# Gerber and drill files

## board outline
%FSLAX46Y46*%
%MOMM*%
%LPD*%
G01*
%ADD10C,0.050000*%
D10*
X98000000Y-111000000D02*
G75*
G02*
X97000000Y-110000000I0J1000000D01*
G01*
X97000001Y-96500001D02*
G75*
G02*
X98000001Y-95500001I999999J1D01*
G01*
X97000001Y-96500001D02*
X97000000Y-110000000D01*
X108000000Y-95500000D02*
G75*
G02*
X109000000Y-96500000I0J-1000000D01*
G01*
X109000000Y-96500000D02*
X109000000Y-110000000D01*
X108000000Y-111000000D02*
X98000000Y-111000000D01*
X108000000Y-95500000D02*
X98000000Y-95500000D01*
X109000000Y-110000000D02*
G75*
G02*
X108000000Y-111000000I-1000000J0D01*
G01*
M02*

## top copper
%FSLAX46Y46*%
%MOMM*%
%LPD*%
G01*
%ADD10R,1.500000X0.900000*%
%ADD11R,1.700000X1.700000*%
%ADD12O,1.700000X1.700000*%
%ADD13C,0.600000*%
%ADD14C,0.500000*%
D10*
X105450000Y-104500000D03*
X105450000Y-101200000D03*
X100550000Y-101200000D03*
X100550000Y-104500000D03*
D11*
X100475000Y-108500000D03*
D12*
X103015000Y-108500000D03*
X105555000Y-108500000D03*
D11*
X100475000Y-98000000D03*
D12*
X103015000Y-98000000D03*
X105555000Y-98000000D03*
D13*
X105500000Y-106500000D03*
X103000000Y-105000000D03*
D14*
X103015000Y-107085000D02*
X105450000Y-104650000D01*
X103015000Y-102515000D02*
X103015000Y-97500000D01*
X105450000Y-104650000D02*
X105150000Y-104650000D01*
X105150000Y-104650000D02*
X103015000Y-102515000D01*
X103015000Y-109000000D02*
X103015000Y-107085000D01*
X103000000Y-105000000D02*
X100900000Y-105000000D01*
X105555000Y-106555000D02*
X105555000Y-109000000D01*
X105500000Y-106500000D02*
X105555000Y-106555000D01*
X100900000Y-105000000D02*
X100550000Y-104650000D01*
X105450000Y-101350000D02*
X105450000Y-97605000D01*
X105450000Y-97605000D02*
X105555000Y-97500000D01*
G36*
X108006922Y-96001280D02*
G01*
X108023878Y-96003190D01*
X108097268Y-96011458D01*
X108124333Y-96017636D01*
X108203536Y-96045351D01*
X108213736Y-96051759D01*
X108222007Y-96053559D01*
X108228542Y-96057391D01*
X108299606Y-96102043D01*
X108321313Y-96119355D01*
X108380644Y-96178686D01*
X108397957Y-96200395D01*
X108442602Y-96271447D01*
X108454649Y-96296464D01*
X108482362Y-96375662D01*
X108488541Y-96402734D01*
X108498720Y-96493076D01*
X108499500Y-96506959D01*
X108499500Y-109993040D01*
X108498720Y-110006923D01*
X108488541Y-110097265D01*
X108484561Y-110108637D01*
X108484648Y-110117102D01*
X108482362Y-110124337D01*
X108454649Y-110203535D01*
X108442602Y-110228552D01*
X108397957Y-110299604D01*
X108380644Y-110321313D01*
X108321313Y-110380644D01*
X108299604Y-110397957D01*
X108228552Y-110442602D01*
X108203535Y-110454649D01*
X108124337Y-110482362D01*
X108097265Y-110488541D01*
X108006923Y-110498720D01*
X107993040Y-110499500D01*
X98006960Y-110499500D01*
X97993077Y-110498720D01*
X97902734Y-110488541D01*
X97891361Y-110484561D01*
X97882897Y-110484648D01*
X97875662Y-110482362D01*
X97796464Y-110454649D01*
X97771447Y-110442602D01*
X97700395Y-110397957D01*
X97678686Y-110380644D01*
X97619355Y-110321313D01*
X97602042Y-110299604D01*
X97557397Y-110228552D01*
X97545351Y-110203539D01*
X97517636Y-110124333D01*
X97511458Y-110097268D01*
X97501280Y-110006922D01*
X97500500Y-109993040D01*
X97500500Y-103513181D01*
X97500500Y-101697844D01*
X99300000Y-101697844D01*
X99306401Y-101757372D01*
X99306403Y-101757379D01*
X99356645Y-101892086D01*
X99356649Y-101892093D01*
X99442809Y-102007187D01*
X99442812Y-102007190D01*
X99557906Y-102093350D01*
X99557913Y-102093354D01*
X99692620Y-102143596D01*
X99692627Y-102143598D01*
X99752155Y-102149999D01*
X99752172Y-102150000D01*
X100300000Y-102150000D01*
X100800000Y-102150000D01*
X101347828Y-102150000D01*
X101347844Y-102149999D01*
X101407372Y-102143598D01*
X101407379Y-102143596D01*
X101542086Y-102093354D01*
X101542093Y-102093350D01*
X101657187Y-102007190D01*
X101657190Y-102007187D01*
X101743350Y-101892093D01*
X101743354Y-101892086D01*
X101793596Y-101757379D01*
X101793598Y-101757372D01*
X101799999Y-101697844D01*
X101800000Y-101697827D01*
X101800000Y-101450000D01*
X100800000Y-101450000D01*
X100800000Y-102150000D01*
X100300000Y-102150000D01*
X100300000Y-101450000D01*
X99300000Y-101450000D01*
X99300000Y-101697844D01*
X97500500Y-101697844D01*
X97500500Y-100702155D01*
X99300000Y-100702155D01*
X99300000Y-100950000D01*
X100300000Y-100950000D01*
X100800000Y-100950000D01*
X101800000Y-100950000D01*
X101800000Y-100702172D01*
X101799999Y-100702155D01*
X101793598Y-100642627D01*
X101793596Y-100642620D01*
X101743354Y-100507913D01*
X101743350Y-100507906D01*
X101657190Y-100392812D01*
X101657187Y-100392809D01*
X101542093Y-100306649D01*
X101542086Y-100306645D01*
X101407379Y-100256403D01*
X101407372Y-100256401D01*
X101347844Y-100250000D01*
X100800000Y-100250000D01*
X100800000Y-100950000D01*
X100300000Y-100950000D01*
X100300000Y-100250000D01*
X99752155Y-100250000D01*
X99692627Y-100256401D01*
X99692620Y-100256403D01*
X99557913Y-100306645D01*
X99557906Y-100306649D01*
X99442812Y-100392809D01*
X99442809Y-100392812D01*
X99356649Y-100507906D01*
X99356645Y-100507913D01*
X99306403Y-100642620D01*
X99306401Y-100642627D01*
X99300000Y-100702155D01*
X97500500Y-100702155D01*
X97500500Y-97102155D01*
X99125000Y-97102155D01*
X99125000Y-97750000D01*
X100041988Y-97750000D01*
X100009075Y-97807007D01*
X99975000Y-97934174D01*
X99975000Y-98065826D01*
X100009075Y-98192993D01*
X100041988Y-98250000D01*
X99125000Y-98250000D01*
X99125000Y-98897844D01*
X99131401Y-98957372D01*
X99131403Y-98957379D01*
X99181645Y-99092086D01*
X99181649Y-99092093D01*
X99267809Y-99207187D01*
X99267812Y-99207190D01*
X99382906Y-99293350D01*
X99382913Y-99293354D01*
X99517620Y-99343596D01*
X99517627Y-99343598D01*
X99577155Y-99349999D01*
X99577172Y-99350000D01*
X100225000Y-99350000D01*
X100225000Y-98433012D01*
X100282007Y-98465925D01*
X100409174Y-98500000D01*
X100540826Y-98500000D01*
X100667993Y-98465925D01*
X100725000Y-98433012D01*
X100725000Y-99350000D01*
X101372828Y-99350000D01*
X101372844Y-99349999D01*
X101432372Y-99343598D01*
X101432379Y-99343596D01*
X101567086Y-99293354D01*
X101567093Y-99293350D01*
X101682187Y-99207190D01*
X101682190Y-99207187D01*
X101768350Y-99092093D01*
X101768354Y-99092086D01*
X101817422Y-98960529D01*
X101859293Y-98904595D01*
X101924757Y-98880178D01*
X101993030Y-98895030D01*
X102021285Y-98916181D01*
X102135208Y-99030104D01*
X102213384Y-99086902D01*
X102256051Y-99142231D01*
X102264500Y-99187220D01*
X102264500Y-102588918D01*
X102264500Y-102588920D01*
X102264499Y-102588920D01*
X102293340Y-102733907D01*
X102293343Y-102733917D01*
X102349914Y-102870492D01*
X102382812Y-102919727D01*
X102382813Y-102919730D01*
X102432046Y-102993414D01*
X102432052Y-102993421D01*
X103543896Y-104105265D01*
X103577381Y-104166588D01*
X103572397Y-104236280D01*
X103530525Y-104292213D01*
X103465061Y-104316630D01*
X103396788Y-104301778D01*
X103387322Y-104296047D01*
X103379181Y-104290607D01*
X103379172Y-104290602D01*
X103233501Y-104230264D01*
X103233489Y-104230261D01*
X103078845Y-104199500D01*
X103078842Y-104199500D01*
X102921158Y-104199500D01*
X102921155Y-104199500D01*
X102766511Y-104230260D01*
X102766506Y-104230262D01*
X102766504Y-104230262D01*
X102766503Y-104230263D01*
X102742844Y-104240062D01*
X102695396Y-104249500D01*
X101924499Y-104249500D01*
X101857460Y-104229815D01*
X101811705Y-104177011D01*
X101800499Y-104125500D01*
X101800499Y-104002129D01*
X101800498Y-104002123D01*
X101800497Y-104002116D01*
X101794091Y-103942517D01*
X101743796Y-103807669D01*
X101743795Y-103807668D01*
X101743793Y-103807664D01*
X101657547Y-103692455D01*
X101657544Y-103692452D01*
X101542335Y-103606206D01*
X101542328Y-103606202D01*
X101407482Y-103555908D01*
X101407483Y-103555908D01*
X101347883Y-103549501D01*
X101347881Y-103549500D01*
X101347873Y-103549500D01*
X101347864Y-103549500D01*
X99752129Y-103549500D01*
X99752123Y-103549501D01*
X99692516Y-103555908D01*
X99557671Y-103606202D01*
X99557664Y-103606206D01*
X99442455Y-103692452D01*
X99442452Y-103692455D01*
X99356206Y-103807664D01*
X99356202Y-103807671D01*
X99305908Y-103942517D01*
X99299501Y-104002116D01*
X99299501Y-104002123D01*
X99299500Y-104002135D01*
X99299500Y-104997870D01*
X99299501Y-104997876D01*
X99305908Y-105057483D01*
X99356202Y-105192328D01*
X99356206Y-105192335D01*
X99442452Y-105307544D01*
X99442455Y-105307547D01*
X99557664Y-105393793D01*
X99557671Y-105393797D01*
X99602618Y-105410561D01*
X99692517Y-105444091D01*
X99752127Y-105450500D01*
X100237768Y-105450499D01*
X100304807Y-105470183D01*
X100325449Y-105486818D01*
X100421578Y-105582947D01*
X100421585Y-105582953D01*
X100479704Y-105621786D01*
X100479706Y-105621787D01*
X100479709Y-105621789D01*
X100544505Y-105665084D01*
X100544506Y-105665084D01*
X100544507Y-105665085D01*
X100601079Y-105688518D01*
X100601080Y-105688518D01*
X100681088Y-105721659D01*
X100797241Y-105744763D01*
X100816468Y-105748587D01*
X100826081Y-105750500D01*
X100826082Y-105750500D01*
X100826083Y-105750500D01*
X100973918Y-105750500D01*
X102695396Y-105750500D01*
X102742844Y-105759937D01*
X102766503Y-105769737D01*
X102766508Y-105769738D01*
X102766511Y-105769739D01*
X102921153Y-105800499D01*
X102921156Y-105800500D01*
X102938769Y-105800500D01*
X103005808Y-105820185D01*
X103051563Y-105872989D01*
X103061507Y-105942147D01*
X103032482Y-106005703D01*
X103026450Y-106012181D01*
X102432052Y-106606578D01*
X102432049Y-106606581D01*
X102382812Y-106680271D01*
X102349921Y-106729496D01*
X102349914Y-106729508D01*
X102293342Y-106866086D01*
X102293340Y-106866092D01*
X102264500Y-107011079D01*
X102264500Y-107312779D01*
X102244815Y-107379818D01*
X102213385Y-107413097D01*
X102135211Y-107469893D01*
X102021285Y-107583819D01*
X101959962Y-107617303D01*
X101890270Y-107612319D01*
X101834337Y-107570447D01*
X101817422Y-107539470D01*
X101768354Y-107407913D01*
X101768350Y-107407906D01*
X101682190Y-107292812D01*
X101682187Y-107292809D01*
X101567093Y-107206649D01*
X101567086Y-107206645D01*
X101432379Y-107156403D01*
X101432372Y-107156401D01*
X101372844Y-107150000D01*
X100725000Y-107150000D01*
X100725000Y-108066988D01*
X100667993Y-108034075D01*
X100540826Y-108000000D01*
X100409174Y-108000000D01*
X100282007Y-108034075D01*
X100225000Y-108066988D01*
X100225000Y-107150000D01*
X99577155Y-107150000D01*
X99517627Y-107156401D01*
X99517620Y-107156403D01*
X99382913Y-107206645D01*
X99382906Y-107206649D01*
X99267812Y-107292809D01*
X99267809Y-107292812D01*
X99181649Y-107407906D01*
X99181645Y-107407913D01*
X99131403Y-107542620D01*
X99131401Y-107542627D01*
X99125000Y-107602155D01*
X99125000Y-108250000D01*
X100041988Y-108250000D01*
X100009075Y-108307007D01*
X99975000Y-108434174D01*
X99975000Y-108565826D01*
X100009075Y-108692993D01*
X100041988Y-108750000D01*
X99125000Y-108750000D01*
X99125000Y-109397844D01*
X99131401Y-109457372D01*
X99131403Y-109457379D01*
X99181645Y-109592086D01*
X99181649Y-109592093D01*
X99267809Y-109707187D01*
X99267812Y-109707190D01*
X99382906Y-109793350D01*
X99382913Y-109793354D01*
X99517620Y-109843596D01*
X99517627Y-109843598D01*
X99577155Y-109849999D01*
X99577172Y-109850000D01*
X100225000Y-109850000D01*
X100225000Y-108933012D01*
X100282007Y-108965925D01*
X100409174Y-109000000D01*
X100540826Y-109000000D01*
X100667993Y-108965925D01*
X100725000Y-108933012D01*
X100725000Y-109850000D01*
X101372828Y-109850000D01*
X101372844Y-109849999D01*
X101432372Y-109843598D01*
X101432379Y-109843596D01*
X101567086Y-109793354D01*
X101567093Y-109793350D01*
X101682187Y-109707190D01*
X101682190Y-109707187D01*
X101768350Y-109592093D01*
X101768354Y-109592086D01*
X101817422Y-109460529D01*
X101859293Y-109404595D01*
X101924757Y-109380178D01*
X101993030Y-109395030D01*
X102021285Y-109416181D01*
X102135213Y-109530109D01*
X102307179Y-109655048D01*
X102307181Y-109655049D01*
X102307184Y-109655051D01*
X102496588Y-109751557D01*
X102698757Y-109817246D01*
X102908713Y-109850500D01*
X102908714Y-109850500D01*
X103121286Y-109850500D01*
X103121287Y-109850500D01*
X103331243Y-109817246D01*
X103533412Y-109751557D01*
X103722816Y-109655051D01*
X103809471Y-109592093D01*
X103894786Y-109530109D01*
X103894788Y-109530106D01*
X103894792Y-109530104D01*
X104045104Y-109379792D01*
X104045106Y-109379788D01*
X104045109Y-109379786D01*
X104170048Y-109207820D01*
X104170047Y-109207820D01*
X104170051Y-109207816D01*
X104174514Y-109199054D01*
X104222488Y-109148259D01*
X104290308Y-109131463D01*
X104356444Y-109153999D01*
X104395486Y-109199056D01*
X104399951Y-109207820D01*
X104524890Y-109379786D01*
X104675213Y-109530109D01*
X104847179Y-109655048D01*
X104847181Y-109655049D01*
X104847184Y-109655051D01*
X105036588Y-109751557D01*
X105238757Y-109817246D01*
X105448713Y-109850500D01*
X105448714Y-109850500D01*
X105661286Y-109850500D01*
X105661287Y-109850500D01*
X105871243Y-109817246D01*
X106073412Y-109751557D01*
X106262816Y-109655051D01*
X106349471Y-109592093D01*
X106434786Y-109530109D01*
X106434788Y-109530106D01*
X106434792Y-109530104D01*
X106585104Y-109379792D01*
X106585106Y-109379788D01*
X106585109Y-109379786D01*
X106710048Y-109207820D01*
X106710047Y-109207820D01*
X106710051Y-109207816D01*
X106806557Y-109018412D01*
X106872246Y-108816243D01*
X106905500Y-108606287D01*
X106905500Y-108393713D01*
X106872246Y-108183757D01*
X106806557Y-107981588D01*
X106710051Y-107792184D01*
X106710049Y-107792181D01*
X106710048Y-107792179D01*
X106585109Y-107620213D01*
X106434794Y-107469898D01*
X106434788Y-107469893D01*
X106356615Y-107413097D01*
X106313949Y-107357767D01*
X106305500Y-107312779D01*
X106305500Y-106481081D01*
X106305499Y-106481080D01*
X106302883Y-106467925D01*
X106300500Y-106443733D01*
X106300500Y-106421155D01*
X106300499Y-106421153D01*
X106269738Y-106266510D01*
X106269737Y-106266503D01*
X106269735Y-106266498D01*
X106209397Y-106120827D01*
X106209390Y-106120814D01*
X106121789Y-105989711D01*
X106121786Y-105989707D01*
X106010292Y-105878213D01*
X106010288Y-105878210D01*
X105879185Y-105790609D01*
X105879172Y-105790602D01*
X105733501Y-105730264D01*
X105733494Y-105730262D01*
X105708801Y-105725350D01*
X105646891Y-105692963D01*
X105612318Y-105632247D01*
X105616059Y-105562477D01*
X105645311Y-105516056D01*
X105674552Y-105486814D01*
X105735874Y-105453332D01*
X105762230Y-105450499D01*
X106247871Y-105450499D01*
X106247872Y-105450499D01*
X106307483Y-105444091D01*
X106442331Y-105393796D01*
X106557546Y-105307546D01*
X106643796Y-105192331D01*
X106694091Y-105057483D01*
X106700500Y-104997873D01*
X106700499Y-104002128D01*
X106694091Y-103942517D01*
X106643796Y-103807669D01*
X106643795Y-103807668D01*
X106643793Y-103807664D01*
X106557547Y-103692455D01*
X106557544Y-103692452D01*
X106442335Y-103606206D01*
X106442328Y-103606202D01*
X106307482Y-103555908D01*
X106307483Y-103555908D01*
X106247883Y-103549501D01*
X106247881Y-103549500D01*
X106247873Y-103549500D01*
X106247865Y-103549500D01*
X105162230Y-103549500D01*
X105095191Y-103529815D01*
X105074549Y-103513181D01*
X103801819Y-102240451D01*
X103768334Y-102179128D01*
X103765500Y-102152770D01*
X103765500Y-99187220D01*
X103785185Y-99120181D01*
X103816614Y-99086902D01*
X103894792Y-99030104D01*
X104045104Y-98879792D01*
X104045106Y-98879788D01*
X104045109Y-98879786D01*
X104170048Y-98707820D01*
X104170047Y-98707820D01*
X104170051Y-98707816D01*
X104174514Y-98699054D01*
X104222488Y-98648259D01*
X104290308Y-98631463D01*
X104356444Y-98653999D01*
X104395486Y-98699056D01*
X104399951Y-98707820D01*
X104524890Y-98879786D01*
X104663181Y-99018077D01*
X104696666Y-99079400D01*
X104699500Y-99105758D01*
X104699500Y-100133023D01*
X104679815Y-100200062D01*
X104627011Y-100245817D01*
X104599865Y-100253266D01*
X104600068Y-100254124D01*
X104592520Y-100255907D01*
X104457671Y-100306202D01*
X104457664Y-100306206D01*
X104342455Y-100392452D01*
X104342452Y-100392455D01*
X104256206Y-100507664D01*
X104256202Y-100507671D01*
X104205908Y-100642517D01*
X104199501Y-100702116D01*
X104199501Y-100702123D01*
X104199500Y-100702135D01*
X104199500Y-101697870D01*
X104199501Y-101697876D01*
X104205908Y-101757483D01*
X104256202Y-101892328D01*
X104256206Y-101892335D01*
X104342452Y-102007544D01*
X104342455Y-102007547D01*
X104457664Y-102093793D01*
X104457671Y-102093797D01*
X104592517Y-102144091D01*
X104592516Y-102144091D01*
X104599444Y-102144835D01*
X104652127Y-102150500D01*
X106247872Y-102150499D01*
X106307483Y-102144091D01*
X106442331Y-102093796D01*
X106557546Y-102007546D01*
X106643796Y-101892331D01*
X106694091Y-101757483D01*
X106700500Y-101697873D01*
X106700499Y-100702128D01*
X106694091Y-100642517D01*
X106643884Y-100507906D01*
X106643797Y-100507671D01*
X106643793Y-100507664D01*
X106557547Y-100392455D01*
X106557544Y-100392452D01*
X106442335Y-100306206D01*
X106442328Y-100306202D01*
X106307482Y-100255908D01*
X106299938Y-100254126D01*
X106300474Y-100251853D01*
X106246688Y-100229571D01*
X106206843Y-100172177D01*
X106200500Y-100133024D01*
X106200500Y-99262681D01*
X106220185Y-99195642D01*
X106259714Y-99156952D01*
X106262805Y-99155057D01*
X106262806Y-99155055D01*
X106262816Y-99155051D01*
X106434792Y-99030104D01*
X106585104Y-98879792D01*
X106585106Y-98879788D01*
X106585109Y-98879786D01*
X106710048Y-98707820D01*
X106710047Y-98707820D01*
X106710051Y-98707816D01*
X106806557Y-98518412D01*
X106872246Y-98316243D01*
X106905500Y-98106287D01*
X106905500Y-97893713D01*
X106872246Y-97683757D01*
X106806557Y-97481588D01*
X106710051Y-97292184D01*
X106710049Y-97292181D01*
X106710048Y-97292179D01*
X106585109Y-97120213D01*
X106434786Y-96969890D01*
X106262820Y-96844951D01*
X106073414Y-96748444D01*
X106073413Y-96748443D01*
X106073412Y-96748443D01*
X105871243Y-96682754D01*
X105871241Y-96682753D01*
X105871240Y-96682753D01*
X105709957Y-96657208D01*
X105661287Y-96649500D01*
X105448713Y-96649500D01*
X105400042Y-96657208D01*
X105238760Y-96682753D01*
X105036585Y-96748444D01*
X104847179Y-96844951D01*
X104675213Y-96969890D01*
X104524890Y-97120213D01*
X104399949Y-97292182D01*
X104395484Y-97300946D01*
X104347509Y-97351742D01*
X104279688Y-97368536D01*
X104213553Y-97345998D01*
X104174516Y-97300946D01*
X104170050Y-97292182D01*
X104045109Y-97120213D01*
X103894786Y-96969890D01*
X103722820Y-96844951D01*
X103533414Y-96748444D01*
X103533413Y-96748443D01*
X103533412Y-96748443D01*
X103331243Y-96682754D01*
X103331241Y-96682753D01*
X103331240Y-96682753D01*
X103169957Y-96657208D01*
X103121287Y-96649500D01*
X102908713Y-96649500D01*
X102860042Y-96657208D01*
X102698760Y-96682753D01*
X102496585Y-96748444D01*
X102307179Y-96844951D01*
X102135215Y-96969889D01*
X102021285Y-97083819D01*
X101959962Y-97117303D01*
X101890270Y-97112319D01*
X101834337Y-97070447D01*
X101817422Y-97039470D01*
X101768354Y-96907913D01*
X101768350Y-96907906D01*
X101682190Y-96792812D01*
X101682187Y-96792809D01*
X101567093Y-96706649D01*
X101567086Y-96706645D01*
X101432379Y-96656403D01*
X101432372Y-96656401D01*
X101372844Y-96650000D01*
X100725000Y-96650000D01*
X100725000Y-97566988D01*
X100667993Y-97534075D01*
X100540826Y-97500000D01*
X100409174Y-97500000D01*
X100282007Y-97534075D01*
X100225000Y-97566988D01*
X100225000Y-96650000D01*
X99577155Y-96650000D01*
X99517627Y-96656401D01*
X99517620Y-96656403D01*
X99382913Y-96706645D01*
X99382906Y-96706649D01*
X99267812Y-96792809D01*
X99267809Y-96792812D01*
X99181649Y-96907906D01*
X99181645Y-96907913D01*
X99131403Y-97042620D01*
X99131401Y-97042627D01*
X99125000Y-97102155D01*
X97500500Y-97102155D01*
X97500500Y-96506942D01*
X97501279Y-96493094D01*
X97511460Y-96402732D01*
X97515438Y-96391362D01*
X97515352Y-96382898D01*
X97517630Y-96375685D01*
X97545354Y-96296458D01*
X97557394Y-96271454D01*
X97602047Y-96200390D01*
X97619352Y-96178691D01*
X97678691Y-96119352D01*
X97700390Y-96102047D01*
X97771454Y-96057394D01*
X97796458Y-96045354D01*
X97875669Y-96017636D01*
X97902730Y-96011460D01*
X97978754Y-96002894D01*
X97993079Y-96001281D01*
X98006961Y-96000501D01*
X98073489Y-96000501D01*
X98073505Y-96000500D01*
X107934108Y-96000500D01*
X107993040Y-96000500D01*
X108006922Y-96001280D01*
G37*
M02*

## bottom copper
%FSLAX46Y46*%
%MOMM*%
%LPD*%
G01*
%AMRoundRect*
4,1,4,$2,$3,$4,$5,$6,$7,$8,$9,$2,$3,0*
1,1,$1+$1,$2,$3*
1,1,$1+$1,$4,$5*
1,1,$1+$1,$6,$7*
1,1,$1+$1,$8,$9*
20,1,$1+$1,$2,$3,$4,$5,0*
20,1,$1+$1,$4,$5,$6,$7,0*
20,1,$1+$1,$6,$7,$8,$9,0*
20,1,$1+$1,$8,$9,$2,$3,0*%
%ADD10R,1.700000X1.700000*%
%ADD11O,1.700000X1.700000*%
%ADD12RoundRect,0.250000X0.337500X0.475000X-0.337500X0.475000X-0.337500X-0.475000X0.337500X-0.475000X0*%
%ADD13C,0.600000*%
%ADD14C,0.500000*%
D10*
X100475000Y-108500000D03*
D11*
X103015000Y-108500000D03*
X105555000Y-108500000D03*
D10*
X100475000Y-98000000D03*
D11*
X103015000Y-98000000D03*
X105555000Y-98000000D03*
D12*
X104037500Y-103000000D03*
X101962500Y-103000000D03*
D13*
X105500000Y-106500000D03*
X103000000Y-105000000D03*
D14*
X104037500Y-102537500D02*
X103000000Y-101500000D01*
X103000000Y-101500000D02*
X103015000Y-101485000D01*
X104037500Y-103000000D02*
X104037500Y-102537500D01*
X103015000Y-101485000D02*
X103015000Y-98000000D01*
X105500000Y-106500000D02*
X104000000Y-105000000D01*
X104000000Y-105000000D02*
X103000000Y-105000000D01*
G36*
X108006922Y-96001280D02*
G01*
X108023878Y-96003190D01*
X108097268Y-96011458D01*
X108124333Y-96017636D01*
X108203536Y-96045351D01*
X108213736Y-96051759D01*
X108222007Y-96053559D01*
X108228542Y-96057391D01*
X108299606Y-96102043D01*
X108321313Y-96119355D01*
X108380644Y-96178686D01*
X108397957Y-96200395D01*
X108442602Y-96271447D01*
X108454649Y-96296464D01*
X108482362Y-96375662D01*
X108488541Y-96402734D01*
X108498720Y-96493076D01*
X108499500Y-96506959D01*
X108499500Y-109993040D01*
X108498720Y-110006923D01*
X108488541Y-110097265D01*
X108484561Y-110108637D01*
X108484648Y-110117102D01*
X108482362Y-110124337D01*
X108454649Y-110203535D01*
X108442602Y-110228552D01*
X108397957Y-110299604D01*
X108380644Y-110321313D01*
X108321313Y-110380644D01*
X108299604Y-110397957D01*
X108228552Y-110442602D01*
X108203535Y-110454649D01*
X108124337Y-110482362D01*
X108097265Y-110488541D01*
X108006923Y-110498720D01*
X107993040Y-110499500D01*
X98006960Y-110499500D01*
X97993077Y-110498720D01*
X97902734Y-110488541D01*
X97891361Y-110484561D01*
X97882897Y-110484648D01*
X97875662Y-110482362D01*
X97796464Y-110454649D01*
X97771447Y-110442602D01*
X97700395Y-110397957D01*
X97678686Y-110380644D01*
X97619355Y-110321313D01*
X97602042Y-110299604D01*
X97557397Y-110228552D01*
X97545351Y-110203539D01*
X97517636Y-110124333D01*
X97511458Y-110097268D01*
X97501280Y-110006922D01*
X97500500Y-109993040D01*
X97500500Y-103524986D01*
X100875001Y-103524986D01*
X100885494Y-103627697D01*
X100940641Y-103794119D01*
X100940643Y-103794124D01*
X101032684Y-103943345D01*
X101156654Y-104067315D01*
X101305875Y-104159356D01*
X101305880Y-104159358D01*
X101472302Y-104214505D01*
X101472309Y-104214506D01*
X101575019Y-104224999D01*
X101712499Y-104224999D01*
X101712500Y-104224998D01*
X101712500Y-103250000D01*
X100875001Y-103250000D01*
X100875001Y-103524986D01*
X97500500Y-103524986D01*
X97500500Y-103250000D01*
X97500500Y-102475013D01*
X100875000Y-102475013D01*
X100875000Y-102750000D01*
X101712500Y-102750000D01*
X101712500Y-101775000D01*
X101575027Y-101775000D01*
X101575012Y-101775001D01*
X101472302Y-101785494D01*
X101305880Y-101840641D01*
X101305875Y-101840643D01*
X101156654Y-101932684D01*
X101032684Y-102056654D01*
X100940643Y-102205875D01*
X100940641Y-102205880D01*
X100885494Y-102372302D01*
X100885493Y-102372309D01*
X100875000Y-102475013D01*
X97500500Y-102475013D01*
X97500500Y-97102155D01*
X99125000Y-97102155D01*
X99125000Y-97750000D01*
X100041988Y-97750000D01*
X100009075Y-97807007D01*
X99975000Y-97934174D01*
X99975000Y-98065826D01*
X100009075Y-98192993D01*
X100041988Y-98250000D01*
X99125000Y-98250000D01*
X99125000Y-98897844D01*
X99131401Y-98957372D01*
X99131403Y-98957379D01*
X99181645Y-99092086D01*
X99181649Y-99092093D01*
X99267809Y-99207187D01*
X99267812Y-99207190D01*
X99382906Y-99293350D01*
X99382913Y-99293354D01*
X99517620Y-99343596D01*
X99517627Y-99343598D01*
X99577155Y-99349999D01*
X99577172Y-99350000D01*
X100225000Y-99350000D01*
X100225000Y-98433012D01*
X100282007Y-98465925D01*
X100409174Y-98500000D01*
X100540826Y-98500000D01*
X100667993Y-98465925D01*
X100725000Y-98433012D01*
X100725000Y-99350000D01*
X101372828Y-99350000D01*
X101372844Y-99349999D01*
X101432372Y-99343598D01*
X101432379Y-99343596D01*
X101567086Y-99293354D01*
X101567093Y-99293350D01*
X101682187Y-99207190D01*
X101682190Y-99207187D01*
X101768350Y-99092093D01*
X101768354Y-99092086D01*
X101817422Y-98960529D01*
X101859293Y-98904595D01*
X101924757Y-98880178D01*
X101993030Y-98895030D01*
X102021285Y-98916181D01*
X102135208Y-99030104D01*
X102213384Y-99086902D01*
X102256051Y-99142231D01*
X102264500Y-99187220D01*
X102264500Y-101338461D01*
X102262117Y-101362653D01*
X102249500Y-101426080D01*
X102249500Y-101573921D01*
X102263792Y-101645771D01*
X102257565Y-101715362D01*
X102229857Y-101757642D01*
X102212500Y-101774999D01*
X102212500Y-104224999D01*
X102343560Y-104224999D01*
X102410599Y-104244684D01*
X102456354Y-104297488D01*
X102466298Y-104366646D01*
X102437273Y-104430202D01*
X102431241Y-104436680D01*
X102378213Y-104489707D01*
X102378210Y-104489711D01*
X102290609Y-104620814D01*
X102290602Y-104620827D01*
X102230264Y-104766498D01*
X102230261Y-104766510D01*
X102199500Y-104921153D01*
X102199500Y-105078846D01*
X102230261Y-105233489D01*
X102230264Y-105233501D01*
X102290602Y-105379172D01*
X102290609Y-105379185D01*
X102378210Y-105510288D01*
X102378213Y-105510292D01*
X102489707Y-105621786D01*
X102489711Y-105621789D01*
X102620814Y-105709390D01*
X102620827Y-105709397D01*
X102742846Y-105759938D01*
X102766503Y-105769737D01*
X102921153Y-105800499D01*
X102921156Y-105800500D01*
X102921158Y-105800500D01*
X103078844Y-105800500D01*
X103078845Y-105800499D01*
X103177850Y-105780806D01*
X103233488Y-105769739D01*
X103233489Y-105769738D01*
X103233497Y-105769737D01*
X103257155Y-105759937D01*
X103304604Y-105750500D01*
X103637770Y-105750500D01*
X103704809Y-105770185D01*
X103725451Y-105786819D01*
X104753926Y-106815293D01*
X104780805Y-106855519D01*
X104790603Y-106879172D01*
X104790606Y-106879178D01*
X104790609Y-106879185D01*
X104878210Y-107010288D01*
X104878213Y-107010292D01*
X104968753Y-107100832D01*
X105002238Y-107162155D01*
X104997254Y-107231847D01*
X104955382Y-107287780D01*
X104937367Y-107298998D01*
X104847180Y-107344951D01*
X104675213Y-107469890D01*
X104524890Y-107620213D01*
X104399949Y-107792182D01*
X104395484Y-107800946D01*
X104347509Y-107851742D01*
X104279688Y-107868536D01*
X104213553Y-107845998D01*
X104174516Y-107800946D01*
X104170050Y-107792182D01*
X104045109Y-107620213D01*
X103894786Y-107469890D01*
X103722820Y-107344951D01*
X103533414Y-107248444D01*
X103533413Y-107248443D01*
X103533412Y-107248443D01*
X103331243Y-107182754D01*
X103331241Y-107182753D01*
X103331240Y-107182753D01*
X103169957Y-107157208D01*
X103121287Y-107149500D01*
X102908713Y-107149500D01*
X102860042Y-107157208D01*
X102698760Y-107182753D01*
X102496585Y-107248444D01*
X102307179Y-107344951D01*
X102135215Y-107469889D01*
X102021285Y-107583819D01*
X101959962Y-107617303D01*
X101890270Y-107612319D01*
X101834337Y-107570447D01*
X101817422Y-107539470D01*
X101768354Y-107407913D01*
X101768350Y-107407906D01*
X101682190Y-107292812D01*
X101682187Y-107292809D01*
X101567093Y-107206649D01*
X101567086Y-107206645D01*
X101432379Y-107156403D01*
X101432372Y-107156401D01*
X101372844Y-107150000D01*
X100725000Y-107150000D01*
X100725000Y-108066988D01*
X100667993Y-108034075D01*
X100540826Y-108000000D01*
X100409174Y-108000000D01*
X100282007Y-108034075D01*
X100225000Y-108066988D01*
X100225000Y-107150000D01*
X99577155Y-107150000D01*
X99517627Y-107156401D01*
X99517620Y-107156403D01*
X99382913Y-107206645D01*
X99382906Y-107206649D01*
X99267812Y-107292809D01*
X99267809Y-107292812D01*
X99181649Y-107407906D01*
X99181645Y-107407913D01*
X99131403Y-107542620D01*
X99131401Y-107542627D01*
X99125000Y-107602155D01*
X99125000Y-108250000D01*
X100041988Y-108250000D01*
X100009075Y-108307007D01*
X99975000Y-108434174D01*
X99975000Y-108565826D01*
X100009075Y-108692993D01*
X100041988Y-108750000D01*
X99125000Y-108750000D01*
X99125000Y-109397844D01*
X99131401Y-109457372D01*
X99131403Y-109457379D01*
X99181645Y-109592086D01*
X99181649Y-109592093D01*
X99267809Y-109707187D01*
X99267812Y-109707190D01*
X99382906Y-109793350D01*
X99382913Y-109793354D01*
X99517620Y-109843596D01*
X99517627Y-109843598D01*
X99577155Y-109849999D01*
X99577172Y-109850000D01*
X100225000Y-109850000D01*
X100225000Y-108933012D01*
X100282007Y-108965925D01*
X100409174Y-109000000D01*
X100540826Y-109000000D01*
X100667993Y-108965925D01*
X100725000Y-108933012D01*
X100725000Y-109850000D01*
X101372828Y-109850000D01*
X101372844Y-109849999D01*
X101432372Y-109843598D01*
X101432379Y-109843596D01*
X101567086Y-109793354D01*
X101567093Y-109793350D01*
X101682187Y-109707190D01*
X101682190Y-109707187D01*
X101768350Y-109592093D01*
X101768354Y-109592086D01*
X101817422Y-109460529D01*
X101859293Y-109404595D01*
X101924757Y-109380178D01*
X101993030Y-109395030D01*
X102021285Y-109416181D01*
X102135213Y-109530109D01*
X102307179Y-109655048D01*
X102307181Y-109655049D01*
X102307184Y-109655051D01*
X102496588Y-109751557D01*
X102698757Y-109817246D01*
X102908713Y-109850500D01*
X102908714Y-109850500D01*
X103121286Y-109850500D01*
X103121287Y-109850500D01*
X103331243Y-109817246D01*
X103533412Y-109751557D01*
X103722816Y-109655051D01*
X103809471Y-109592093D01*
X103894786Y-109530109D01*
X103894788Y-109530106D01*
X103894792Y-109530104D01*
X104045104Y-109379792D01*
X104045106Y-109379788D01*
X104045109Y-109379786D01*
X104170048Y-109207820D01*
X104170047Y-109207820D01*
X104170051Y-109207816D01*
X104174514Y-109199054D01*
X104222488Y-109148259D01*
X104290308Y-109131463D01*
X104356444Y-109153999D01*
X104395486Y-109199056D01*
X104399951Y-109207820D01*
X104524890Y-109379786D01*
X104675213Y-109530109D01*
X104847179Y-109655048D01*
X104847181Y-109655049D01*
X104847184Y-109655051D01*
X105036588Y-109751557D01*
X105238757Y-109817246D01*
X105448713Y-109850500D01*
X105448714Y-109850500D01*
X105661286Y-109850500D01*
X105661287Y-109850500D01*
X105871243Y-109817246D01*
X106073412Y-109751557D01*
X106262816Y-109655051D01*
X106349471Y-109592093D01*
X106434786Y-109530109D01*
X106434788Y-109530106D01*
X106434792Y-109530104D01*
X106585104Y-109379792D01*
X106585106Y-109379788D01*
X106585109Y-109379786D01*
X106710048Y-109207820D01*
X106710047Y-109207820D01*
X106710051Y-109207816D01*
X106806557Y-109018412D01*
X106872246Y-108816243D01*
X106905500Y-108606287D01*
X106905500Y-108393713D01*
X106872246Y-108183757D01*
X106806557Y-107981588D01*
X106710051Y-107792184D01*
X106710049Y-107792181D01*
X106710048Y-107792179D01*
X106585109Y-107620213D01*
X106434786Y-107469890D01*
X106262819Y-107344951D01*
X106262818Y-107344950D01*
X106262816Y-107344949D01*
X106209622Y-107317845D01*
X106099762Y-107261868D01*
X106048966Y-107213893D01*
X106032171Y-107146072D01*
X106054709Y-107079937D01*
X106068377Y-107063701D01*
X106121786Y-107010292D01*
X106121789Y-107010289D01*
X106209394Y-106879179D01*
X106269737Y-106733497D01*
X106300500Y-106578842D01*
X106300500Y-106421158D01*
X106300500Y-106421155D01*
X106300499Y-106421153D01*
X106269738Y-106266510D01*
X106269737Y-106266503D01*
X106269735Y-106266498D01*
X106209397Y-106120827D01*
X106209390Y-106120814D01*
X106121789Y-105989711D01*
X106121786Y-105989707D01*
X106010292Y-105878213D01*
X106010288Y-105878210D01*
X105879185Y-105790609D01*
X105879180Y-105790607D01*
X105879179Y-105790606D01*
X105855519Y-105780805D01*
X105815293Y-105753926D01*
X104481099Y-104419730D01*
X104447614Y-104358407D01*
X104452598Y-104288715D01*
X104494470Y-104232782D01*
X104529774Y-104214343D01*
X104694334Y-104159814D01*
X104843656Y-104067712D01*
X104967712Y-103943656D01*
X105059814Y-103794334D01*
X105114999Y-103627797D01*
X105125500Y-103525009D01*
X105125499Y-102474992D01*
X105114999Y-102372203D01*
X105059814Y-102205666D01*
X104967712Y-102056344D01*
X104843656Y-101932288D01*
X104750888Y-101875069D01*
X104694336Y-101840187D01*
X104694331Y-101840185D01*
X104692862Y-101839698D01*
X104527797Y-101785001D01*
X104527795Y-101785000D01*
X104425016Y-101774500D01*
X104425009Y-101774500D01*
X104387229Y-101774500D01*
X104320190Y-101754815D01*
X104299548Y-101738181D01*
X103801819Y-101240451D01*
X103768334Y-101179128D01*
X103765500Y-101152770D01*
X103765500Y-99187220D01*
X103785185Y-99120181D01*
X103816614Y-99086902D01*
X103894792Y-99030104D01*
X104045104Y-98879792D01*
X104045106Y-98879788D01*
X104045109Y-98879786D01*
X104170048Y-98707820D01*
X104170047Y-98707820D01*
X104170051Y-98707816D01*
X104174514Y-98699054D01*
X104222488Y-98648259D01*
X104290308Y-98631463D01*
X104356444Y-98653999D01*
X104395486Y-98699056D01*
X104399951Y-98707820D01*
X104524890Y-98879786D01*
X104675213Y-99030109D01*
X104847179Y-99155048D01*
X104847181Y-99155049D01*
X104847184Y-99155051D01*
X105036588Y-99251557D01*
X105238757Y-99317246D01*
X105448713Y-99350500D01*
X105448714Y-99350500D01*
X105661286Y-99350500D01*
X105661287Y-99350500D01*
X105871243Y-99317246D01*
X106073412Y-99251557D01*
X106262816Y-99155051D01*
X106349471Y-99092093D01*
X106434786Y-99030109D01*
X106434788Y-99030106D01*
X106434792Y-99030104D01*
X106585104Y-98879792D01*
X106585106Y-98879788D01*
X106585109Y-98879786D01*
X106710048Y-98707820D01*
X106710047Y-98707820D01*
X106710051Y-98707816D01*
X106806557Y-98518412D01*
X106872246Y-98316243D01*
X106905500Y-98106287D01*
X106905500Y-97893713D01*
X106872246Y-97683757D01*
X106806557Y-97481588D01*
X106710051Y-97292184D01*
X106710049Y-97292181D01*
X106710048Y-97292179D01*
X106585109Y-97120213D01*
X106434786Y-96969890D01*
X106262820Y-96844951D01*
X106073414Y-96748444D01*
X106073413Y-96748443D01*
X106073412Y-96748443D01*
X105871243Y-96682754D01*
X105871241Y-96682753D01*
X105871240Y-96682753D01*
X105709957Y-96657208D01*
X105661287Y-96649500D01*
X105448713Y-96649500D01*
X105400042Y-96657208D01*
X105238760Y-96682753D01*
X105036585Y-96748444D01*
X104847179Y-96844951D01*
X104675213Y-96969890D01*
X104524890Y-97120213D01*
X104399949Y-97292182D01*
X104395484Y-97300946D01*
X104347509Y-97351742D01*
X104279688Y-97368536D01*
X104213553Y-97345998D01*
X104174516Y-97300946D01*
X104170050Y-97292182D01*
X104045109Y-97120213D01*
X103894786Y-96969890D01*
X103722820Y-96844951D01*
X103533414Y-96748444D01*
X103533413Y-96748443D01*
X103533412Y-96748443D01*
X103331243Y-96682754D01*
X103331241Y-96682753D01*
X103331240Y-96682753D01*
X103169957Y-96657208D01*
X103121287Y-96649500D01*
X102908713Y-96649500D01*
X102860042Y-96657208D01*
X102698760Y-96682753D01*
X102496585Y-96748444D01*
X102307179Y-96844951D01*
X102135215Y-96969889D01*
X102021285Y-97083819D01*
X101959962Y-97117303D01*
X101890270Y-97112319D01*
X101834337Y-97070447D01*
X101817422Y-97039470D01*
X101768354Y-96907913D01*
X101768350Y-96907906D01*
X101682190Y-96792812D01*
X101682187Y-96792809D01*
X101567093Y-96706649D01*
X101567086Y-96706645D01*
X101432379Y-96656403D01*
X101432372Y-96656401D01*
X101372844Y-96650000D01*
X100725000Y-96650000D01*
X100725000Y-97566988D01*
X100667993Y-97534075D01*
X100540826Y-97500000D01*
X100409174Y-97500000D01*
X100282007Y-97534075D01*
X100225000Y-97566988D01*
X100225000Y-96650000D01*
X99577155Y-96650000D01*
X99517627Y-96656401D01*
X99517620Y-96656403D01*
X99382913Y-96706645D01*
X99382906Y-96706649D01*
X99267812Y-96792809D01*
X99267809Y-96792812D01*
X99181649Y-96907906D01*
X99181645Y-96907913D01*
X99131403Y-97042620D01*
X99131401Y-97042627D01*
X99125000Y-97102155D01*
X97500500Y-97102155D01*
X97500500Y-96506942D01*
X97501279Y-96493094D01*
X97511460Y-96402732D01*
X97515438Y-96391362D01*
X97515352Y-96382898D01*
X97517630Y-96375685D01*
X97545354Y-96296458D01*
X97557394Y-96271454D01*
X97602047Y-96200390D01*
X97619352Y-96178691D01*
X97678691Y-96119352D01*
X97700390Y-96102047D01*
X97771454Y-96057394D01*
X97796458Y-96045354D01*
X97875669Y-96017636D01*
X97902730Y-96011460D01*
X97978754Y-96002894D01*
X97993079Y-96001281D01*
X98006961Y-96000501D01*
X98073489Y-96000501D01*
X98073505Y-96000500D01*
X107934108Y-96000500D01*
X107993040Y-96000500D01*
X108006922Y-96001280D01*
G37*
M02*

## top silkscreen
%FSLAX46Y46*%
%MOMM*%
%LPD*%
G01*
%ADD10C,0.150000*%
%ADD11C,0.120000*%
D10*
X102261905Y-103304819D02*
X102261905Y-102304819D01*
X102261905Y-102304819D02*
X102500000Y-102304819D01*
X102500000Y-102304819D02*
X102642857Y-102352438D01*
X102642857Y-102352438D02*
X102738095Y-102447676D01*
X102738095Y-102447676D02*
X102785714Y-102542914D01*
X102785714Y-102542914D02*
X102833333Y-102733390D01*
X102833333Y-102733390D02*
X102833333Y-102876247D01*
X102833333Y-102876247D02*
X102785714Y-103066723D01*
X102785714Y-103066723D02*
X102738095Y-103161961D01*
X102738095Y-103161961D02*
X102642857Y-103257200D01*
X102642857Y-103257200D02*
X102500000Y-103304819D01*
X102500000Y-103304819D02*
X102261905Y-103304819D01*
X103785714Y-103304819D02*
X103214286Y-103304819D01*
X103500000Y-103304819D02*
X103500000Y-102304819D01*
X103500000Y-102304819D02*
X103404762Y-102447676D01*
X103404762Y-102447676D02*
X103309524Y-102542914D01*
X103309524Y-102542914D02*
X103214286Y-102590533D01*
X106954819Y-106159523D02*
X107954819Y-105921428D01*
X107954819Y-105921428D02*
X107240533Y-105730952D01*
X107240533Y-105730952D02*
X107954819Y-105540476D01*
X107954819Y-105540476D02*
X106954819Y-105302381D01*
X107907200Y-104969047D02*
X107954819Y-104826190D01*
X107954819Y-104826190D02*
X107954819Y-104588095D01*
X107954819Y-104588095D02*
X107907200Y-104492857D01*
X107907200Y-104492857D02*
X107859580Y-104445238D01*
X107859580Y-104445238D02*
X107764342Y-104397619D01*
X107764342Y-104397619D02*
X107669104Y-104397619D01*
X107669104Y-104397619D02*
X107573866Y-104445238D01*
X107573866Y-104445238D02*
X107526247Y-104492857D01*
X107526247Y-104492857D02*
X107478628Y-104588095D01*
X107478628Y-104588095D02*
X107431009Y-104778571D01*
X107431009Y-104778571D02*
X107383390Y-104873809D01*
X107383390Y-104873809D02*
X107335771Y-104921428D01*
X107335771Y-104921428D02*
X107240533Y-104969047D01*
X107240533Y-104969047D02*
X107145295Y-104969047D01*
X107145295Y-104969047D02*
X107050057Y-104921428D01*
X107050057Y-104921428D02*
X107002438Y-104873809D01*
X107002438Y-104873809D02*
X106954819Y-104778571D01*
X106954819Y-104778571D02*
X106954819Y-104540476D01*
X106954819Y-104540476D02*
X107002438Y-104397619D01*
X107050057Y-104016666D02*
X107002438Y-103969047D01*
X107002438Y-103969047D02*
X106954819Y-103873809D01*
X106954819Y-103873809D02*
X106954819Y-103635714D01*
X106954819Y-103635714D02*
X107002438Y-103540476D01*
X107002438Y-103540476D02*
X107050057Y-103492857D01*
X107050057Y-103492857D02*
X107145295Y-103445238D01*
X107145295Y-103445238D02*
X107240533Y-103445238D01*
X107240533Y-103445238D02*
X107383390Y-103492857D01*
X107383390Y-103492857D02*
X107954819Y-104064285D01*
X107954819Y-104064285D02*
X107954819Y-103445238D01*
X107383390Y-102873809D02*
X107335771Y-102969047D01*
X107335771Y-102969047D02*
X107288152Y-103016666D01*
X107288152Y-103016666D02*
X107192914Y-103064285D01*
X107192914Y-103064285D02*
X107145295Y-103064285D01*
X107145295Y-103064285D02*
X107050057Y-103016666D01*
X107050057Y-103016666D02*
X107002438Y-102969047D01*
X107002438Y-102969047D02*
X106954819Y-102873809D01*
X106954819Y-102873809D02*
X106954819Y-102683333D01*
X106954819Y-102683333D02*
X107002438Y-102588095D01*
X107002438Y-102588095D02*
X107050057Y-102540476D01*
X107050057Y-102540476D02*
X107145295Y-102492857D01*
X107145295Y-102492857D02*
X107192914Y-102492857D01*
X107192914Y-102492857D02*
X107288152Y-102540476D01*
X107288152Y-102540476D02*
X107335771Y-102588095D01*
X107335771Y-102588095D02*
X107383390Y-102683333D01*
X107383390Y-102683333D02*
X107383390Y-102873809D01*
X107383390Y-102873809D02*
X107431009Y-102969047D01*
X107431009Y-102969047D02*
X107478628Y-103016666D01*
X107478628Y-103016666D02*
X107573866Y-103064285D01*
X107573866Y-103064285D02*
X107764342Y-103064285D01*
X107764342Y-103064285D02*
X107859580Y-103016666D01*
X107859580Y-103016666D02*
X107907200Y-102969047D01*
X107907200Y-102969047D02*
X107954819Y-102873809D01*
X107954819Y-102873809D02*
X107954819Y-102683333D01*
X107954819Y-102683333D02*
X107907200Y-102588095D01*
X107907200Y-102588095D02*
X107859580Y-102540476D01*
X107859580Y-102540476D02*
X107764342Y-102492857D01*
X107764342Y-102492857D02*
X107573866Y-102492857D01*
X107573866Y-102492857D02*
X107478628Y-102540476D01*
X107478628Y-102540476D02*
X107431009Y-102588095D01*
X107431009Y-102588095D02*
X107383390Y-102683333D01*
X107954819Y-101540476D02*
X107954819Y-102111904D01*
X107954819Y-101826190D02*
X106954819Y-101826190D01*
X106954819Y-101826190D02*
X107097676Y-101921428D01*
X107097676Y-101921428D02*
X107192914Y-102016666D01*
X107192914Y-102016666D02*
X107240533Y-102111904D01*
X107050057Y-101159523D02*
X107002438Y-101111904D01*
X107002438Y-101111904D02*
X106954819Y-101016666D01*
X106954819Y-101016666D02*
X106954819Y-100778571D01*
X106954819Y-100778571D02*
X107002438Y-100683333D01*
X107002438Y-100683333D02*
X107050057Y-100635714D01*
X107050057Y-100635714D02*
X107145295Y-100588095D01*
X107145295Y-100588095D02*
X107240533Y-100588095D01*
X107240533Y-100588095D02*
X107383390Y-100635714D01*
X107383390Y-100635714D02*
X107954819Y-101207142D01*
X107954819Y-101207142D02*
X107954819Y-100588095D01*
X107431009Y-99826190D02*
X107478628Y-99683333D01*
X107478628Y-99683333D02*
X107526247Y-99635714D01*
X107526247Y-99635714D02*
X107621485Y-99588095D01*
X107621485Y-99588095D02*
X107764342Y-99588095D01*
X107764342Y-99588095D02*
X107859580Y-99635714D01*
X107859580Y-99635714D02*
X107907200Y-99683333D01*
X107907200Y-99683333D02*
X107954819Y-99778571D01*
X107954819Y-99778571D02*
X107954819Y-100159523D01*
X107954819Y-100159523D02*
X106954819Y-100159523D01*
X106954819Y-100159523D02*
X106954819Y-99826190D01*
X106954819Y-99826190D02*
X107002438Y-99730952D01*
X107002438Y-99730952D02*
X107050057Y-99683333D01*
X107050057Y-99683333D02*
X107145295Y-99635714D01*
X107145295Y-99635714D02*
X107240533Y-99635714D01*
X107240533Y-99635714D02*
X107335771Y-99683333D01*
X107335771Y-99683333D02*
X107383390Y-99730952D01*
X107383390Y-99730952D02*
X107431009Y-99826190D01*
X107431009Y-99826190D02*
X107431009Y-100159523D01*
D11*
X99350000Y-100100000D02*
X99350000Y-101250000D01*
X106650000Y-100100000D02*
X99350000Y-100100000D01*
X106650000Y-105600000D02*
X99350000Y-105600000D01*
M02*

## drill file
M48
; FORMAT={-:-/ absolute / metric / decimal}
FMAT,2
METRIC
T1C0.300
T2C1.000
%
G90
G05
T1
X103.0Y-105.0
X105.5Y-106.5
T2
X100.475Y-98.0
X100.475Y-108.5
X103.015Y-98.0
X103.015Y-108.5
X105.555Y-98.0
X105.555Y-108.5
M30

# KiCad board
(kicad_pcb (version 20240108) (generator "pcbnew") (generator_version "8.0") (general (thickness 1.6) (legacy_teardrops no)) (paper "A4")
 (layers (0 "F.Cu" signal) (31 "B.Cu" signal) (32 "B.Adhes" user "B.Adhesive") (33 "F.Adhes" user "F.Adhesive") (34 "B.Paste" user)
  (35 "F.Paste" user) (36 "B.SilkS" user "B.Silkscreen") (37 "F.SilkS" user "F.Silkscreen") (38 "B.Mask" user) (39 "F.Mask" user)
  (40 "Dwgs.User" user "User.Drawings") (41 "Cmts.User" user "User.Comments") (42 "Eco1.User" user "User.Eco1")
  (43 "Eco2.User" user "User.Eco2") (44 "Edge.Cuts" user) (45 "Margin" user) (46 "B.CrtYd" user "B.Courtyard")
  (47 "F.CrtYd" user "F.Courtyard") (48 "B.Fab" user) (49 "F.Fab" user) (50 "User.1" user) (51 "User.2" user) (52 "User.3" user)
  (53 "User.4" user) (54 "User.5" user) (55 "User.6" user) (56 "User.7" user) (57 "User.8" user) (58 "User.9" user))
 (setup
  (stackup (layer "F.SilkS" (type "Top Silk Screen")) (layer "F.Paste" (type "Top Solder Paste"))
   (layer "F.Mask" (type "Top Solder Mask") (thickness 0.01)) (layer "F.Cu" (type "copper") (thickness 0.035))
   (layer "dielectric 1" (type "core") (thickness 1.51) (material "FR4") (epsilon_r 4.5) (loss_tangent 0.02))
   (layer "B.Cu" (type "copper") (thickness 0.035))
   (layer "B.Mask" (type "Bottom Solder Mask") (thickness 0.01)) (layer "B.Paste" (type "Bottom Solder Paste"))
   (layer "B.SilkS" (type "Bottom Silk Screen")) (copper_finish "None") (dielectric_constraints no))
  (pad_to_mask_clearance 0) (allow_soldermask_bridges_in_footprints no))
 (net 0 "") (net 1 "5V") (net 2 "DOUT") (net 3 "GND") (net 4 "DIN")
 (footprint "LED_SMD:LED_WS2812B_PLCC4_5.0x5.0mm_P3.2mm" (layer "F.Cu") (at 103 102.85 180)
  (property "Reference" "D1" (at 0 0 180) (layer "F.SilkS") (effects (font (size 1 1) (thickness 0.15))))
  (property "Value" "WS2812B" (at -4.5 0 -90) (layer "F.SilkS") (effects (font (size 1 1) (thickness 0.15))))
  (fp_line (start 3.65 2.75) (end 3.65 1.6) (stroke (width 0.12) (type solid)) (layer "F.SilkS"))
  (fp_line (start -3.65 2.75) (end 3.65 2.75) (stroke (width 0.12) (type solid)) (layer "F.SilkS"))
  (fp_line (start -3.65 -2.75) (end 3.65 -2.75) (stroke (width 0.12) (type solid)) (layer "F.SilkS"))
  (pad "1" smd rect (at -2.45 -1.65 180) (size 1.5 0.9) (layers "F.Cu" "F.Paste" "F.Mask") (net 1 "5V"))
  (pad "2" smd rect (at -2.45 1.65 180) (size 1.5 0.9) (layers "F.Cu" "F.Paste" "F.Mask") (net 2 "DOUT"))
  (pad "3" smd rect (at 2.45 1.65 180) (size 1.5 0.9) (layers "F.Cu" "F.Paste" "F.Mask") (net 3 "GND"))
  (pad "4" smd rect (at 2.45 -1.65 180) (size 1.5 0.9) (layers "F.Cu" "F.Paste" "F.Mask") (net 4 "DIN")))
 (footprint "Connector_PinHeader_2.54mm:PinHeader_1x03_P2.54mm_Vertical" (layer "B.Cu") (at 100.475 108.5 -90)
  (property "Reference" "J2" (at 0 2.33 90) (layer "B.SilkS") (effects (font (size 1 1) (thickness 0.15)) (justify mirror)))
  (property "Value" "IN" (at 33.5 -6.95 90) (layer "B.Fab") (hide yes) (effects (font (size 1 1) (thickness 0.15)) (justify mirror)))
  (pad "1" thru_hole rect (at 0 0 270) (size 1.7 1.7) (drill 1) (layers "*.Cu" "*.Mask") (remove_unused_layers no) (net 3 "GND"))
  (pad "2" thru_hole oval (at 0 -2.54 270) (size 1.7 1.7) (drill 1) (layers "*.Cu" "*.Mask") (remove_unused_layers no) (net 1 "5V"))
  (pad "3" thru_hole oval (at 0 -5.08 270) (size 1.7 1.7) (drill 1) (layers "*.Cu" "*.Mask") (remove_unused_layers no) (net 4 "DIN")))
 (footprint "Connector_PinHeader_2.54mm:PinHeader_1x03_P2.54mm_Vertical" (layer "B.Cu") (at 100.475 98 -90)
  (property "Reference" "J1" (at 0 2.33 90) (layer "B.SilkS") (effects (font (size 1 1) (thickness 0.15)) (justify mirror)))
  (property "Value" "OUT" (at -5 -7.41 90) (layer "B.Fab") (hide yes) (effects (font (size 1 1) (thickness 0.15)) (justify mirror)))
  (pad "1" thru_hole rect (at 0 0 270) (size 1.7 1.7) (drill 1) (layers "*.Cu" "*.Mask") (remove_unused_layers no) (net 3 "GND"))
  (pad "2" thru_hole oval (at 0 -2.54 270) (size 1.7 1.7) (drill 1) (layers "*.Cu" "*.Mask") (remove_unused_layers no) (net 1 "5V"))
  (pad "3" thru_hole oval (at 0 -5.08 270) (size 1.7 1.7) (drill 1) (layers "*.Cu" "*.Mask") (remove_unused_layers no) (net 2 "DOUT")))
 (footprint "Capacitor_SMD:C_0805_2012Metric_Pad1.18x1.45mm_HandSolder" (layer "B.Cu") (at 103 103 180)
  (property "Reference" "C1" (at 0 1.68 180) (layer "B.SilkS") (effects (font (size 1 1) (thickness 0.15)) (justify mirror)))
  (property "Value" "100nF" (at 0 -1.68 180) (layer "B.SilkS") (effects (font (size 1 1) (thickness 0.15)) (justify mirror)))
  (pad "1" smd roundrect (at -1.0375 0 180) (size 1.175 1.45) (layers "B.Cu" "B.Paste" "B.Mask") (roundrect_rratio 0.212766) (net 1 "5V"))
  (pad "2" smd roundrect (at 1.0375 0 180) (size 1.175 1.45) (layers "B.Cu" "B.Paste" "B.Mask") (roundrect_rratio 0.212766) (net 3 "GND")))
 (gr_arc (start 98 111) (mid 97.292893 110.707107) (end 97 110) (stroke (width 0.05) (type default)) (layer "Edge.Cuts"))
 (gr_arc (start 97.000001 96.500001) (mid 97.292894 95.792894) (end 98.000001 95.500001) (stroke (width 0.05) (type default))
  (layer "Edge.Cuts"))
 (gr_line (start 97.000001 96.500001) (end 97 110) (stroke (width 0.05) (type default)) (layer "Edge.Cuts"))
 (gr_arc (start 108 95.5) (mid 108.707107 95.792893) (end 109 96.5) (stroke (width 0.05) (type default)) (layer "Edge.Cuts"))
 (gr_line (start 109 96.5) (end 109 110) (stroke (width 0.05) (type default)) (layer "Edge.Cuts"))
 (gr_line (start 108 111) (end 98 111) (stroke (width 0.05) (type default)) (layer "Edge.Cuts"))
 (gr_line (start 108 95.5) (end 98 95.5) (stroke (width 0.05) (type default)) (layer "Edge.Cuts"))
 (gr_arc (start 109 110) (mid 108.707107 110.707107) (end 108 111) (stroke (width 0.05) (type default)) (layer "Edge.Cuts"))
 (segment (start 103.015 107.085) (end 105.45 104.65) (width 0.5) (layer "F.Cu") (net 1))
 (segment (start 103.015 102.515) (end 103.015 97.5) (width 0.5) (layer "F.Cu") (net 1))
 (segment (start 105.45 104.65) (end 105.15 104.65) (width 0.5) (layer "F.Cu") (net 1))
 (segment (start 105.15 104.65) (end 103.015 102.515) (width 0.5) (layer "F.Cu") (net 1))
 (segment (start 103.015 109) (end 103.015 107.085) (width 0.5) (layer "F.Cu") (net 1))
 (segment (start 104.0375 102.5375) (end 103 101.5) (width 0.5) (layer "B.Cu") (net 1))
 (segment (start 103 101.5) (end 103.015 101.485) (width 0.5) (layer "B.Cu") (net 1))
 (segment (start 104.0375 103) (end 104.0375 102.5375) (width 0.5) (layer "B.Cu") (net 1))
 (segment (start 103.015 101.485) (end 103.015 98) (width 0.5) (layer "B.Cu") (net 1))
 (segment (start 103 105) (end 100.9 105) (width 0.5) (layer "F.Cu") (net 4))
 (segment (start 105.555 106.555) (end 105.555 109) (width 0.5) (layer "F.Cu") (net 4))
 (segment (start 105.5 106.5) (end 105.555 106.555) (width 0.5) (layer "F.Cu") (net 4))
 (segment (start 100.9 105) (end 100.55 104.65) (width 0.5) (layer "F.Cu") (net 4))
 (via (at 105.5 106.5) (size 0.6) (drill 0.3) (layers "F.Cu" "B.Cu") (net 4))
 (via (at 103 105) (size 0.6) (drill 0.3) (layers "F.Cu" "B.Cu") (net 4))
 (segment (start 105.5 106.5) (end 104 105) (width 0.5) (layer "B.Cu") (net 4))
 (segment (start 104 105) (end 103 105) (width 0.5) (layer "B.Cu") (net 4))
 (segment (start 105.45 101.35) (end 105.45 97.605) (width 0.5) (layer "F.Cu") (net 2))
 (segment (start 105.45 97.605) (end 105.555 97.5) (width 0.5) (layer "F.Cu") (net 2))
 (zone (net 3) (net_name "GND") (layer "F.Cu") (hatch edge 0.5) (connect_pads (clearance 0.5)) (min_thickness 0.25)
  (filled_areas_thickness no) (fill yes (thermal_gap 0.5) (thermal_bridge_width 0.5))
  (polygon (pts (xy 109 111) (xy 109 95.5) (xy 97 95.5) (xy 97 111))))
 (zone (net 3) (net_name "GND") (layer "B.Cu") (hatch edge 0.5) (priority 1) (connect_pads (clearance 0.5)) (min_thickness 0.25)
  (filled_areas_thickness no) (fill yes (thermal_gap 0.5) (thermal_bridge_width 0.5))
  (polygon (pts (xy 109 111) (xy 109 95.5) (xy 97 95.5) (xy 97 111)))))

